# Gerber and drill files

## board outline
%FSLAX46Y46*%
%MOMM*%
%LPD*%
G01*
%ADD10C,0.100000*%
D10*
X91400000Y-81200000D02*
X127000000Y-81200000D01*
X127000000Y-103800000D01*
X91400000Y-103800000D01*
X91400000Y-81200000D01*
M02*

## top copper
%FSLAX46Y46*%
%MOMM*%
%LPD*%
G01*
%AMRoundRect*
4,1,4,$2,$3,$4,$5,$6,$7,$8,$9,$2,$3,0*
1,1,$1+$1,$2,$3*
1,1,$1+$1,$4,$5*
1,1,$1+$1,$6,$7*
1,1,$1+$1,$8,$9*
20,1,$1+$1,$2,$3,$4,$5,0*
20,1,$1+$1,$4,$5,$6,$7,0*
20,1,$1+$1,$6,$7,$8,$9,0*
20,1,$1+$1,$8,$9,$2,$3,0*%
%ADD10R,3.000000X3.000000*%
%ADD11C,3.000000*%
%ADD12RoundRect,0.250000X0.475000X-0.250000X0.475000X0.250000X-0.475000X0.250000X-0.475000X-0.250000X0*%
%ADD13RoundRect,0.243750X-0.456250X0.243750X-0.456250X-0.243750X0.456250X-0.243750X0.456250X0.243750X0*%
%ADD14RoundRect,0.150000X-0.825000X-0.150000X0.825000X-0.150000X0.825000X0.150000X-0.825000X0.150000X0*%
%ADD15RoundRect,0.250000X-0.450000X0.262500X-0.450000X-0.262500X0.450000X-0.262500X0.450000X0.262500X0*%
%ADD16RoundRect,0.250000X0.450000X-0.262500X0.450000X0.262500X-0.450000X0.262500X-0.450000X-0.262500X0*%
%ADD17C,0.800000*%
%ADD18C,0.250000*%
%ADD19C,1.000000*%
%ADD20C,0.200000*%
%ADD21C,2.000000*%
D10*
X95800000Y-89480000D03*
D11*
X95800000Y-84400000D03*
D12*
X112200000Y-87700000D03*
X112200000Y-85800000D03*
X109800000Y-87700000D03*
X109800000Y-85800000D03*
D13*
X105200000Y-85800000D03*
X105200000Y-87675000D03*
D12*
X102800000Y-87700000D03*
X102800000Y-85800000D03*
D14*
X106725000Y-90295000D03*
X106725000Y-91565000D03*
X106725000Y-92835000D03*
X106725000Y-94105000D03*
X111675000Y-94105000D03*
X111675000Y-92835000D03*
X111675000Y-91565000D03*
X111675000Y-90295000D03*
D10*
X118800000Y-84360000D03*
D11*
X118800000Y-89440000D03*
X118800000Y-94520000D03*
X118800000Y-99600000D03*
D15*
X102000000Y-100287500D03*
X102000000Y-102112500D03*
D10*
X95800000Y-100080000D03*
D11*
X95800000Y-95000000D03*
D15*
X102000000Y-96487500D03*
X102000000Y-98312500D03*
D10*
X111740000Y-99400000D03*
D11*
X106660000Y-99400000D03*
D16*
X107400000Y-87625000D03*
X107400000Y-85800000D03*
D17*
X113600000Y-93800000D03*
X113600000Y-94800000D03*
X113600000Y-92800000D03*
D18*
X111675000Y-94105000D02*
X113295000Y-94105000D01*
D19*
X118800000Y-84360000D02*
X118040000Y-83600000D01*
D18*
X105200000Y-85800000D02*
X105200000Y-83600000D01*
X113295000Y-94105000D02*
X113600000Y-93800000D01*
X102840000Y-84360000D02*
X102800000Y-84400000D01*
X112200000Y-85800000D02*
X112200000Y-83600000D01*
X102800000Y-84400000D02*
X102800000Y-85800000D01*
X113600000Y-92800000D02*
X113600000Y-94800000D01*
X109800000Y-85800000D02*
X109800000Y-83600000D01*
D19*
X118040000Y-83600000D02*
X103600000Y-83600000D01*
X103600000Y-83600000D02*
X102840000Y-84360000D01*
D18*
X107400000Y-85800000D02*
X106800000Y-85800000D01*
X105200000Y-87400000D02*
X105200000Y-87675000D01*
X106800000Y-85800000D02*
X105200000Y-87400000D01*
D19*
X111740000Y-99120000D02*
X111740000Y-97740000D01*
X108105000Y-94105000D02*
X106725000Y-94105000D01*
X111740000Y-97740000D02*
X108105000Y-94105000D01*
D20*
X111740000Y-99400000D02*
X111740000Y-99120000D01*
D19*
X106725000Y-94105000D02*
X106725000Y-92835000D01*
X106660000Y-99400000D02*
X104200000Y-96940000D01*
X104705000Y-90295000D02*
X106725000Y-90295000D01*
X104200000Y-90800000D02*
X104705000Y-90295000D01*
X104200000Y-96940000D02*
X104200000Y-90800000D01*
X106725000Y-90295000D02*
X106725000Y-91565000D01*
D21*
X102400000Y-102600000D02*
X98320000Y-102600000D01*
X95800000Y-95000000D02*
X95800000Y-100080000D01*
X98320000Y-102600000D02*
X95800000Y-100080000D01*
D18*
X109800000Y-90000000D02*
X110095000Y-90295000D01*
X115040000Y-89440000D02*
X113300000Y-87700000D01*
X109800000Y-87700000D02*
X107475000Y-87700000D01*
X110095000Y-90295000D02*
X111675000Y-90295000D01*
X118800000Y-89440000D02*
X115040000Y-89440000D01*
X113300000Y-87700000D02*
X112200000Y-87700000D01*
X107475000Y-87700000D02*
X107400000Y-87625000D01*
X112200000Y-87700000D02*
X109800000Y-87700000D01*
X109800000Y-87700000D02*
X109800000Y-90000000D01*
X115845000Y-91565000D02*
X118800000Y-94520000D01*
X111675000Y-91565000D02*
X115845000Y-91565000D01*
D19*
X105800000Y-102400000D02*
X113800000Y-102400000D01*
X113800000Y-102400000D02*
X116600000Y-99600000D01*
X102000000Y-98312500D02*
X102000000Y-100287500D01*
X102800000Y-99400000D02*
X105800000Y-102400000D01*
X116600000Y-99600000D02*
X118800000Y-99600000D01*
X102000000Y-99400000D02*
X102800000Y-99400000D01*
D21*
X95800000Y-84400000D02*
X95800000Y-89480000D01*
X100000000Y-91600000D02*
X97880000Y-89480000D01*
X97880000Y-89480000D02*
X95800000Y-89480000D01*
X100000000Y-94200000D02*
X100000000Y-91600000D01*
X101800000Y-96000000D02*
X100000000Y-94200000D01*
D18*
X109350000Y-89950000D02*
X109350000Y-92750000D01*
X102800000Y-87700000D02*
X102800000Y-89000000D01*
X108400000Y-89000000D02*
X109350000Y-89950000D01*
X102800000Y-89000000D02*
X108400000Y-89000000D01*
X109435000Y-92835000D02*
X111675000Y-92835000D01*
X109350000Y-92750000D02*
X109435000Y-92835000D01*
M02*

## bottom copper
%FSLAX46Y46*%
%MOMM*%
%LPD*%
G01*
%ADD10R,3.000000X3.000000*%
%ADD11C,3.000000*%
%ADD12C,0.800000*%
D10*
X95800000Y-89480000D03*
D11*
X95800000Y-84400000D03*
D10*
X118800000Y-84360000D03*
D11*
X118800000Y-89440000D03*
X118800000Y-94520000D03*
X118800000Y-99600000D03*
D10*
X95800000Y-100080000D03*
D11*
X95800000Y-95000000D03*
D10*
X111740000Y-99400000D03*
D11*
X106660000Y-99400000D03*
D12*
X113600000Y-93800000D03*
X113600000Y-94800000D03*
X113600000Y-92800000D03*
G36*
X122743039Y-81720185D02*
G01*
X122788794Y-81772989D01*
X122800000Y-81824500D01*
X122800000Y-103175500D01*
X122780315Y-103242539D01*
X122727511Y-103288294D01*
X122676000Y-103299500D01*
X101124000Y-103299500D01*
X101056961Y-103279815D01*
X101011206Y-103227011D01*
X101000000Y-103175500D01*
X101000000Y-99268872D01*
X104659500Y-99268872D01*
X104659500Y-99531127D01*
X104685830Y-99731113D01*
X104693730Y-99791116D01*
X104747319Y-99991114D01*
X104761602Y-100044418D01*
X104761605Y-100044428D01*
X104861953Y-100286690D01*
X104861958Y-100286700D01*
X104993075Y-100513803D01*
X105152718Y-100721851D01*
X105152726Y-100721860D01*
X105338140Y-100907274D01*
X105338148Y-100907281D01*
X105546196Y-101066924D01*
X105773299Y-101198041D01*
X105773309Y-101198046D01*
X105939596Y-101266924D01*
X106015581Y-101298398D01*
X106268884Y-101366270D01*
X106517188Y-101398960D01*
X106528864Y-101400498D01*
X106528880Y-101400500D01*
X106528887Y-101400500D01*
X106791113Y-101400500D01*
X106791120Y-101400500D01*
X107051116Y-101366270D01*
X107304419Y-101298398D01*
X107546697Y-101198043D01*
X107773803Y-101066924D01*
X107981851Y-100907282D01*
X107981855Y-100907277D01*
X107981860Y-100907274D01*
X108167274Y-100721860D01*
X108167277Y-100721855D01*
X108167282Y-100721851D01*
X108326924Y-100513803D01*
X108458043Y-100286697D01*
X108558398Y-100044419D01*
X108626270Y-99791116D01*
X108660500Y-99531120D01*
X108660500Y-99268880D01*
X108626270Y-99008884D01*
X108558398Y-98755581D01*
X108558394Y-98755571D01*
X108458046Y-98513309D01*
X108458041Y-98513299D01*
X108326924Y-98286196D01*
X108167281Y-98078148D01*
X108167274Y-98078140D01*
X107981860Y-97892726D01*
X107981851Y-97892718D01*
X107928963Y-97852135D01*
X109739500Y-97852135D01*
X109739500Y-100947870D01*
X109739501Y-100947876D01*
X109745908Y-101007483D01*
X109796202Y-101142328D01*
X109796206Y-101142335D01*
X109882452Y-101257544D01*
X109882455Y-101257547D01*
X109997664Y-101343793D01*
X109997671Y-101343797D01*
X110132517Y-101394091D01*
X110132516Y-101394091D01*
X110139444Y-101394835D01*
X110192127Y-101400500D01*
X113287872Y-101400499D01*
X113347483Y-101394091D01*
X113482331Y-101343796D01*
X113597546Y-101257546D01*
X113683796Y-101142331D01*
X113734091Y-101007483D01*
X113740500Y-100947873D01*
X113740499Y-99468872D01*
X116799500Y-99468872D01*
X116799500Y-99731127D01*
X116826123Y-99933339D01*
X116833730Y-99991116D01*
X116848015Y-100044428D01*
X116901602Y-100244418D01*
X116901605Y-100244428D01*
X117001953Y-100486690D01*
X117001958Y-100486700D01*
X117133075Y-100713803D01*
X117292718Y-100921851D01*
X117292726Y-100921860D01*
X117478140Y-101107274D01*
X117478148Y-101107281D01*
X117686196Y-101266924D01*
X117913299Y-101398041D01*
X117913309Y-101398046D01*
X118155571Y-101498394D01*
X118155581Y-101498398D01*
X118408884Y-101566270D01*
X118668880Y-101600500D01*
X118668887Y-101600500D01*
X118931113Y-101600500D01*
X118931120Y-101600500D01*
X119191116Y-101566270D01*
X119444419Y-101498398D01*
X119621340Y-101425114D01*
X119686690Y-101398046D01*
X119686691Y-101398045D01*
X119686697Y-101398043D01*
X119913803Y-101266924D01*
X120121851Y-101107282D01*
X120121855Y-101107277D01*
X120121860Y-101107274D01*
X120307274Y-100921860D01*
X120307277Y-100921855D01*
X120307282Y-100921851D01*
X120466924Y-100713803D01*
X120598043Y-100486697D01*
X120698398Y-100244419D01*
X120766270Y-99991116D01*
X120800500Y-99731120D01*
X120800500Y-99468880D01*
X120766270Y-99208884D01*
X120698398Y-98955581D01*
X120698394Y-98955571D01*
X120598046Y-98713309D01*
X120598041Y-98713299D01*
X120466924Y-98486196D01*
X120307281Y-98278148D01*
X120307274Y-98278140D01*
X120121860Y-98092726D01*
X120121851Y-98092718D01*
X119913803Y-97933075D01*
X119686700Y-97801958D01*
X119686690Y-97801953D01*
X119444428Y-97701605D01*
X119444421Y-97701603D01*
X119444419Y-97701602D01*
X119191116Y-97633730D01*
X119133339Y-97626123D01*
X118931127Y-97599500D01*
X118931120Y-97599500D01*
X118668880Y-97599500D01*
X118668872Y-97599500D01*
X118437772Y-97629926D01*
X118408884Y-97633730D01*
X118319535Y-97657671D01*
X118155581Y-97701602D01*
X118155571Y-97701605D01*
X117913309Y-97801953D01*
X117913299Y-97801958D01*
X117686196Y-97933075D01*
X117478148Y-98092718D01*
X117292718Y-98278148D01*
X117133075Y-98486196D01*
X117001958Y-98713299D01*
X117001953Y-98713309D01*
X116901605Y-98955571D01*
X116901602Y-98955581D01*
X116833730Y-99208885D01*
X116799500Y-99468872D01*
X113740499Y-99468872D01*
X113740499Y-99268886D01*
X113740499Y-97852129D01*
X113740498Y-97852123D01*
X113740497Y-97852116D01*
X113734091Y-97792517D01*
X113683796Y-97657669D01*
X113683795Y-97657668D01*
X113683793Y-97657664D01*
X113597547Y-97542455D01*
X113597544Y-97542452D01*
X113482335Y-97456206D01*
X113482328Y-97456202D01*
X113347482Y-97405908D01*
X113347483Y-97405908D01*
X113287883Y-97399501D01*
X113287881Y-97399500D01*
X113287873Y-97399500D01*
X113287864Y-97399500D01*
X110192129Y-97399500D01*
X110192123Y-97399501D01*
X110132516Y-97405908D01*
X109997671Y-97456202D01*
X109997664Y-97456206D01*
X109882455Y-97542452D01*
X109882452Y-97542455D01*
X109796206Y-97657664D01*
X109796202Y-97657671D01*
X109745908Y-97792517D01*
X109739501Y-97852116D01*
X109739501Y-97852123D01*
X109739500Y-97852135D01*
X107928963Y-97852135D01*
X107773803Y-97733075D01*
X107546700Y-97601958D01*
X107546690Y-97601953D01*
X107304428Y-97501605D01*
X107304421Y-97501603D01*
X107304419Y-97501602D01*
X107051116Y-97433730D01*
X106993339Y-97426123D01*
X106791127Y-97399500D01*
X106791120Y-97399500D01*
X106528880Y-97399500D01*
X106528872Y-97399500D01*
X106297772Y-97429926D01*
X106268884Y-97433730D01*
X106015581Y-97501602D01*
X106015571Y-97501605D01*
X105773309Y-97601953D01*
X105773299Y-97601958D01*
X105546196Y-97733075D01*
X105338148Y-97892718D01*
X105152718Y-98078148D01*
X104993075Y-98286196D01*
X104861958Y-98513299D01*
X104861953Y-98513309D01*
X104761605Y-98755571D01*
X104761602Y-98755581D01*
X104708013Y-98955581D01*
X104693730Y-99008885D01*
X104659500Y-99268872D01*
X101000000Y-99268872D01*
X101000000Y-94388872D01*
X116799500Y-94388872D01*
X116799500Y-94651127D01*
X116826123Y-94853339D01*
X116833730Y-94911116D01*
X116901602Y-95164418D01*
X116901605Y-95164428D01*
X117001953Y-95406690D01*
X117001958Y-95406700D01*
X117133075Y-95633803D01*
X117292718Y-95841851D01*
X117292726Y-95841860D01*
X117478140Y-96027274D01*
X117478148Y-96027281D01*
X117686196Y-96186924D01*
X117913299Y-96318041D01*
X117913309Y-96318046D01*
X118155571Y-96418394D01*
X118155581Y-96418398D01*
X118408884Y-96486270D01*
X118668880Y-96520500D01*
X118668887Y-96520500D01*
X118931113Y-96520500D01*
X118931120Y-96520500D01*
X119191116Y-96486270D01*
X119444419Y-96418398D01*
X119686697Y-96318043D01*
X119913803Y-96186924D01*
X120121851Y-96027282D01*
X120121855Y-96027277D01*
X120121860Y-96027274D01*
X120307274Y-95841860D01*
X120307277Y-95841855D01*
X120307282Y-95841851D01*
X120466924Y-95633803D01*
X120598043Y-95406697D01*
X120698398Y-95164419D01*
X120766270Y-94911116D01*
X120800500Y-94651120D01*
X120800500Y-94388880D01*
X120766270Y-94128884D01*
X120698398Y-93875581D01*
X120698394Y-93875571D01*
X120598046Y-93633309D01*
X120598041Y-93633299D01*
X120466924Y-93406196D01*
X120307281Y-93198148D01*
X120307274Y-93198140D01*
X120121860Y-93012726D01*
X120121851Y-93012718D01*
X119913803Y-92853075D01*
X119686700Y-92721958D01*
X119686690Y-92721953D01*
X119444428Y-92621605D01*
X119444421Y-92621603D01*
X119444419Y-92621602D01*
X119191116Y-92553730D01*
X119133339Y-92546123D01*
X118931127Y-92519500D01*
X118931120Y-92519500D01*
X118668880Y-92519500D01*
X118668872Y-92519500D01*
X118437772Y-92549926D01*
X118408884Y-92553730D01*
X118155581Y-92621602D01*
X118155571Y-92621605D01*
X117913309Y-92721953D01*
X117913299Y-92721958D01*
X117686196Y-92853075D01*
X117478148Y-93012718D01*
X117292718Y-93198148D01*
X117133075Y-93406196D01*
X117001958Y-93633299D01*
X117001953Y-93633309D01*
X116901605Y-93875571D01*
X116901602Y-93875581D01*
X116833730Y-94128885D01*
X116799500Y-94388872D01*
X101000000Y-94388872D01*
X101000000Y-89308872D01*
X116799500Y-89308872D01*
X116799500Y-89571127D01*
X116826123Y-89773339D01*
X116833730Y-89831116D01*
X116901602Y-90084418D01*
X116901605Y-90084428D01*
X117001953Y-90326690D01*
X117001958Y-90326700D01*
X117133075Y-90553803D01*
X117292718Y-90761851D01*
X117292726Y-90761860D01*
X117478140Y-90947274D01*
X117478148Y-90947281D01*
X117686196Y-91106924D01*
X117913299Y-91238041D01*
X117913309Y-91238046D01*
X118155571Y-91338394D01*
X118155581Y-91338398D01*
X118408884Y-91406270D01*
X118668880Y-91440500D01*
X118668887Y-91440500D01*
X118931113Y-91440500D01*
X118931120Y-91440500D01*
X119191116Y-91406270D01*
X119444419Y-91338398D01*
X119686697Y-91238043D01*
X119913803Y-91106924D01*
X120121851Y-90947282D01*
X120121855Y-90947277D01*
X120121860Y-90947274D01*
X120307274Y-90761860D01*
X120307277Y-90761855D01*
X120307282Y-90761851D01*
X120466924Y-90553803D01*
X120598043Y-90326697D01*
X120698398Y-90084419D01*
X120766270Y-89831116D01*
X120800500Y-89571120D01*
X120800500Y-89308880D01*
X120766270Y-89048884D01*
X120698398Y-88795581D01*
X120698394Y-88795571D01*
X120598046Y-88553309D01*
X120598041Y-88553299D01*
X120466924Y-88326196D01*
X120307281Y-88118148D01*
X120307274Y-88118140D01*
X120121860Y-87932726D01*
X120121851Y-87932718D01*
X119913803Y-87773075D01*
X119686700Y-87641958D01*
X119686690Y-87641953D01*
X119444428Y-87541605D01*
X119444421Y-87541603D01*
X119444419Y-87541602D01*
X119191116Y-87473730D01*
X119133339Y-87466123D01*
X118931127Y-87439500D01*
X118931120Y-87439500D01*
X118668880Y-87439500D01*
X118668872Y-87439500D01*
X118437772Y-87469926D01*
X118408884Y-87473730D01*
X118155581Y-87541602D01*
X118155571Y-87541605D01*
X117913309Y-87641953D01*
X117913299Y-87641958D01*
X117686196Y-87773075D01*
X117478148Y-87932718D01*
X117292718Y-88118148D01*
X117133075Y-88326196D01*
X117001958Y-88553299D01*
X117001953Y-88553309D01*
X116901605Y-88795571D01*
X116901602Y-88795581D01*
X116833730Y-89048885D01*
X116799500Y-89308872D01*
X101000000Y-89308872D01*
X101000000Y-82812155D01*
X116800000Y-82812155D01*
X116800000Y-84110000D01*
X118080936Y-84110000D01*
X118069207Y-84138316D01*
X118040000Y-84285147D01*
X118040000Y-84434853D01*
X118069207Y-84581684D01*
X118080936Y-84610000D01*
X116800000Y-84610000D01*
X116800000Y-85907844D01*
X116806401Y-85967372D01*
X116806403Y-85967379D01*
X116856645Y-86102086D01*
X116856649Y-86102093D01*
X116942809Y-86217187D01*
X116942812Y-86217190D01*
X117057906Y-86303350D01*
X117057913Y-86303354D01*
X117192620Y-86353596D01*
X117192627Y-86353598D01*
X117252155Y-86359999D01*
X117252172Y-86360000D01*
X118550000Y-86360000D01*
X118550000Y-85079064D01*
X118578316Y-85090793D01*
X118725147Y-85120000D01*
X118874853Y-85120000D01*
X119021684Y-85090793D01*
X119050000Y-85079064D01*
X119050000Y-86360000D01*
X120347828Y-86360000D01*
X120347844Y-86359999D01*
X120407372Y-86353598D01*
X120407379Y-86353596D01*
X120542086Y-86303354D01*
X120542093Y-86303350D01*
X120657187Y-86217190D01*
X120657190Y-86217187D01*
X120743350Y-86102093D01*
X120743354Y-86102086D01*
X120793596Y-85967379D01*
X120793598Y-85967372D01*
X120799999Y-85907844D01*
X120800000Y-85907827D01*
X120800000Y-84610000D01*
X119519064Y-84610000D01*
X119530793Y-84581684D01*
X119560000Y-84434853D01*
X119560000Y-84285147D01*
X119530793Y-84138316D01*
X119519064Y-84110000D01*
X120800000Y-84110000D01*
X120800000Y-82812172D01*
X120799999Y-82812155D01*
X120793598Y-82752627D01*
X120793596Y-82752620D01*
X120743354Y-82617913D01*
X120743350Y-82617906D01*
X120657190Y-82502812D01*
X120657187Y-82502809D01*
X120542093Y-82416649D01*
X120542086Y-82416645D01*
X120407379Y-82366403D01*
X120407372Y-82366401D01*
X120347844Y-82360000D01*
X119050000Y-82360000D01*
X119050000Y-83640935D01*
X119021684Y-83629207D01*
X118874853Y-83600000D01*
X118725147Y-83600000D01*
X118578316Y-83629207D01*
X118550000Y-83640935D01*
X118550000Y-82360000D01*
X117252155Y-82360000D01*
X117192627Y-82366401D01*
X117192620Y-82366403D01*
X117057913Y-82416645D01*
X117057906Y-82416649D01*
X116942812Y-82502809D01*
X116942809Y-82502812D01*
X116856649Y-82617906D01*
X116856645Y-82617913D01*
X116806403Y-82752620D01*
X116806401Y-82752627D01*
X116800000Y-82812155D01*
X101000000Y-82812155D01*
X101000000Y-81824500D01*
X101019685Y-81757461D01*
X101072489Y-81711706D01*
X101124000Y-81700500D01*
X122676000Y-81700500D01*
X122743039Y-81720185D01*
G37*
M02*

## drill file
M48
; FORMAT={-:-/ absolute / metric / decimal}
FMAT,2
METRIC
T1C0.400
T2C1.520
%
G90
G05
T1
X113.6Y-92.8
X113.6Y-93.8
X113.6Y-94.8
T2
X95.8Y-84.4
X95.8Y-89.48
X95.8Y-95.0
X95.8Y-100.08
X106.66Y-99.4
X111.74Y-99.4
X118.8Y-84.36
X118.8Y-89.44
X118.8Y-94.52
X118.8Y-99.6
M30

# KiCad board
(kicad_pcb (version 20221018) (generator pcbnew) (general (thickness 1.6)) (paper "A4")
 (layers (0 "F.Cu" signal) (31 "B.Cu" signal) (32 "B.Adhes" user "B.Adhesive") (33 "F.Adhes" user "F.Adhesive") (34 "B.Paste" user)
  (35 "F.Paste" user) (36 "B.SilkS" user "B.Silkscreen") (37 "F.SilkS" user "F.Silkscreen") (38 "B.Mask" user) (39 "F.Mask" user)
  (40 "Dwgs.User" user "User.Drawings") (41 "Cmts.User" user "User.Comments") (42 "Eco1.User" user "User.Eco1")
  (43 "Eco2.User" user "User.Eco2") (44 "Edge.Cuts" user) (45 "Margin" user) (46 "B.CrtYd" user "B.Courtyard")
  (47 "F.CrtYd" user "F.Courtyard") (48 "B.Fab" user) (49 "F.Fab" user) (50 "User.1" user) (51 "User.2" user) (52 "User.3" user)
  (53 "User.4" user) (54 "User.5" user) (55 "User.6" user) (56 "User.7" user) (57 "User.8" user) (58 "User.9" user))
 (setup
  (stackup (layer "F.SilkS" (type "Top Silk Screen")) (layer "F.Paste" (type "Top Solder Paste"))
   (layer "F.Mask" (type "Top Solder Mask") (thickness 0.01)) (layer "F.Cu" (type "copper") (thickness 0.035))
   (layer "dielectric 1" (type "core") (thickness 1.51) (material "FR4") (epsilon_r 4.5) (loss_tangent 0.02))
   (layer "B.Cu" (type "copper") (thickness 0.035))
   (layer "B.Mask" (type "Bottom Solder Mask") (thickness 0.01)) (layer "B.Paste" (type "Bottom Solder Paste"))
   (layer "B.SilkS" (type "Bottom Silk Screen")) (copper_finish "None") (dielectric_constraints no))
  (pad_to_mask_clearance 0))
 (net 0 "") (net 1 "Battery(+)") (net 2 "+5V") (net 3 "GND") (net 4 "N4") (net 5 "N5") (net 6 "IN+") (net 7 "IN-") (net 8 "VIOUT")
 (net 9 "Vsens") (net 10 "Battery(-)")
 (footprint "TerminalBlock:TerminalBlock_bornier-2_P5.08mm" (layer "F.Cu") (at 95.8 89.48 90)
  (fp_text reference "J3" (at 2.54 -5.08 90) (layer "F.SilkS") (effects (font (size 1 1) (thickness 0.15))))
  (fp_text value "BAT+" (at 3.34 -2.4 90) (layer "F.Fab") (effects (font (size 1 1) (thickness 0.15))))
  (pad "1" thru_hole rect (at 0 0 90) (size 3 3) (drill 1.52) (layers "*.Cu" "*.Mask") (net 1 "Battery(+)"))
  (pad "2" thru_hole circle (at 5.08 0 90) (size 3 3) (drill 1.52) (layers "*.Cu" "*.Mask") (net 1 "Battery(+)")))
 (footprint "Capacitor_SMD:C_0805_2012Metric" (layer "F.Cu") (at 112.2 86.75 90)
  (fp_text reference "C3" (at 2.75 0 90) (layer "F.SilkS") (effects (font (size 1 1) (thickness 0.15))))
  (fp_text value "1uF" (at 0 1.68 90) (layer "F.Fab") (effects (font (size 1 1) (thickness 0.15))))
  (pad "1" smd roundrect (at -0.95 0 90) (size 1 1.45) (layers "F.Cu" "F.Paste" "F.Mask") (roundrect_rratio 0.25) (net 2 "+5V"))
  (pad "2" smd roundrect (at 0.95 0 90) (size 1 1.45) (layers "F.Cu" "F.Paste" "F.Mask") (roundrect_rratio 0.25) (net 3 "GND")))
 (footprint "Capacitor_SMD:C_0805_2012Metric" (layer "F.Cu") (at 109.8 86.75 90)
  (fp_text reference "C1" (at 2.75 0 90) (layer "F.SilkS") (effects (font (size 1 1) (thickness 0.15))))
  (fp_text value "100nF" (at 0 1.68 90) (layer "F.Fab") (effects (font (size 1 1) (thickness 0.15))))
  (pad "1" smd roundrect (at -0.95 0 90) (size 1 1.45) (layers "F.Cu" "F.Paste" "F.Mask") (roundrect_rratio 0.25) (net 2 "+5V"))
  (pad "2" smd roundrect (at 0.95 0 90) (size 1 1.45) (layers "F.Cu" "F.Paste" "F.Mask") (roundrect_rratio 0.25) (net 3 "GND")))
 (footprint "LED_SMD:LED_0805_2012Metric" (layer "F.Cu") (at 105.2 86.7375 -90)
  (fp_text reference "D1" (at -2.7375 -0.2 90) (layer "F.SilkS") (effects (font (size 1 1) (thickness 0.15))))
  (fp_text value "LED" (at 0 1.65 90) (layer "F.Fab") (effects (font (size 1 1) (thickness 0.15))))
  (pad "1" smd roundrect (at -0.9375 0 270) (size 0.975 1.4) (layers "F.Cu" "F.Paste" "F.Mask") (roundrect_rratio 0.25) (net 3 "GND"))
  (pad "2" smd roundrect (at 0.9375 0 270) (size 0.975 1.4) (layers "F.Cu" "F.Paste" "F.Mask") (roundrect_rratio 0.25) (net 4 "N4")))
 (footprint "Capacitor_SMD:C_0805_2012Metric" (layer "F.Cu") (at 102.8 86.75 90)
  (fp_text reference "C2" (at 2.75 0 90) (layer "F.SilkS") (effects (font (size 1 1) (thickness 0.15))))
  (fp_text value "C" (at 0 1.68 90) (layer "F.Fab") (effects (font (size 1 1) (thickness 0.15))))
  (pad "1" smd roundrect (at -0.95 0 90) (size 1 1.45) (layers "F.Cu" "F.Paste" "F.Mask") (roundrect_rratio 0.25) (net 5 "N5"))
  (pad "2" smd roundrect (at 0.95 0 90) (size 1 1.45) (layers "F.Cu" "F.Paste" "F.Mask") (roundrect_rratio 0.25) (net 3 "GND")))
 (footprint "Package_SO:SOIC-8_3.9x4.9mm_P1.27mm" (layer "F.Cu") (at 109.2 92.2)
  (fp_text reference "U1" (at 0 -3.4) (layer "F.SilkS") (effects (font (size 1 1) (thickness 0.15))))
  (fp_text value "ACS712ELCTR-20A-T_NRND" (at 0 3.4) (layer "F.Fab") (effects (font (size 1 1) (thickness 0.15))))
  (pad "1" smd roundrect (at -2.475 -1.905) (size 1.95 0.6) (layers "F.Cu" "F.Paste" "F.Mask") (roundrect_rratio 0.25) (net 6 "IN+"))
  (pad "2" smd roundrect (at -2.475 -0.635) (size 1.95 0.6) (layers "F.Cu" "F.Paste" "F.Mask") (roundrect_rratio 0.25) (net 6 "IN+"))
  (pad "3" smd roundrect (at -2.475 0.635) (size 1.95 0.6) (layers "F.Cu" "F.Paste" "F.Mask") (roundrect_rratio 0.25) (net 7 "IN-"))
  (pad "4" smd roundrect (at -2.475 1.905) (size 1.95 0.6) (layers "F.Cu" "F.Paste" "F.Mask") (roundrect_rratio 0.25) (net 7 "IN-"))
  (pad "5" smd roundrect (at 2.475 1.905) (size 1.95 0.6) (layers "F.Cu" "F.Paste" "F.Mask") (roundrect_rratio 0.25) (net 3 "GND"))
  (pad "6" smd roundrect (at 2.475 0.635) (size 1.95 0.6) (layers "F.Cu" "F.Paste" "F.Mask") (roundrect_rratio 0.25) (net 5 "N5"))
  (pad "7" smd roundrect (at 2.475 -0.635) (size 1.95 0.6) (layers "F.Cu" "F.Paste" "F.Mask") (roundrect_rratio 0.25) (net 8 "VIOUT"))
  (pad "8" smd roundrect (at 2.475 -1.905) (size 1.95 0.6) (layers "F.Cu" "F.Paste" "F.Mask") (roundrect_rratio 0.25) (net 2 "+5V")))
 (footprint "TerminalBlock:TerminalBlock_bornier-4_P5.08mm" (layer "F.Cu") (at 118.8 84.36 -90)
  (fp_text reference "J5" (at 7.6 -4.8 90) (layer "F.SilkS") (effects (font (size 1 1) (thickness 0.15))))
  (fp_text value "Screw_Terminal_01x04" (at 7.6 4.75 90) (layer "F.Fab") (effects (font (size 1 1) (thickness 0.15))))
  (pad "1" thru_hole rect (at 0 0 270) (size 3 3) (drill 1.52) (layers "*.Cu" "*.Mask") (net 3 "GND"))
  (pad "2" thru_hole circle (at 5.08 0 270) (size 3 3) (drill 1.52) (layers "*.Cu" "*.Mask") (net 2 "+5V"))
  (pad "3" thru_hole circle (at 10.16 0 270) (size 3 3) (drill 1.52) (layers "*.Cu" "*.Mask") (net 8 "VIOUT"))
  (pad "4" thru_hole circle (at 15.24 0 270) (size 3 3) (drill 1.52) (layers "*.Cu" "*.Mask") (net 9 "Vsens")))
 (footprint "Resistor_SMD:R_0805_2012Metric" (layer "F.Cu") (at 102 101.2 -90)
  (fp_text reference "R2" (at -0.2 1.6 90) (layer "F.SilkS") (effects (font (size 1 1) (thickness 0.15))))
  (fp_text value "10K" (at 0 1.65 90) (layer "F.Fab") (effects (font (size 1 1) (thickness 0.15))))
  (pad "1" smd roundrect (at -0.9125 0 270) (size 1.025 1.4) (layers "F.Cu" "F.Paste" "F.Mask") (roundrect_rratio 0.243902) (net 9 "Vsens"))
  (pad "2" smd roundrect (at 0.9125 0 270) (size 1.025 1.4) (layers "F.Cu" "F.Paste" "F.Mask") (roundrect_rratio 0.243902)
   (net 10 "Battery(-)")))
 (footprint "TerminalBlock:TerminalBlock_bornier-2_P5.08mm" (layer "F.Cu") (at 95.8 100.08 90)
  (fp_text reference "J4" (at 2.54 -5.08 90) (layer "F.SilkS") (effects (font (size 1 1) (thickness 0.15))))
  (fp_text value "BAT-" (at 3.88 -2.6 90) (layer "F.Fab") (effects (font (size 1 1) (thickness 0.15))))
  (pad "1" thru_hole rect (at 0 0 90) (size 3 3) (drill 1.52) (layers "*.Cu" "*.Mask") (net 10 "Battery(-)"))
  (pad "2" thru_hole circle (at 5.08 0 90) (size 3 3) (drill 1.52) (layers "*.Cu" "*.Mask") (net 10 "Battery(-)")))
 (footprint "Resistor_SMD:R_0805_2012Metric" (layer "F.Cu") (at 102 97.4 -90)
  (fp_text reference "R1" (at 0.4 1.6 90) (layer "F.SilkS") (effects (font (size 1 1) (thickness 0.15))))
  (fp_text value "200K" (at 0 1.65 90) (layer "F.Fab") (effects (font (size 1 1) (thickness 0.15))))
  (pad "1" smd roundrect (at -0.9125 0 270) (size 1.025 1.4) (layers "F.Cu" "F.Paste" "F.Mask") (roundrect_rratio 0.243902)
   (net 1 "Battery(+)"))
  (pad "2" smd roundrect (at 0.9125 0 270) (size 1.025 1.4) (layers "F.Cu" "F.Paste" "F.Mask") (roundrect_rratio 0.243902) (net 9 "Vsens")))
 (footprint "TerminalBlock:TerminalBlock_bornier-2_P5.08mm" (layer "F.Cu") (at 111.74 99.4 180)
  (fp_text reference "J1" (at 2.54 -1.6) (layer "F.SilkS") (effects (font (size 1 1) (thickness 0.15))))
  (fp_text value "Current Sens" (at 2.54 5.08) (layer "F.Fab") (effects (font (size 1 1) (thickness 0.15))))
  (pad "1" thru_hole rect (at 0 0 180) (size 3 3) (drill 1.52) (layers "*.Cu" "*.Mask") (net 7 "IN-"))
  (pad "2" thru_hole circle (at 5.08 0 180) (size 3 3) (drill 1.52) (layers "*.Cu" "*.Mask") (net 6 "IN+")))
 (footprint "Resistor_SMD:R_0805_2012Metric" (layer "F.Cu") (at 107.4 86.7125 90)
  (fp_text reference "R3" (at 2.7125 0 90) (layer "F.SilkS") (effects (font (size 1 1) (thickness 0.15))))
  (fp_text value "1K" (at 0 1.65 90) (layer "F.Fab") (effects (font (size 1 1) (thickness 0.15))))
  (pad "1" smd roundrect (at -0.9125 0 90) (size 1.025 1.4) (layers "F.Cu" "F.Paste" "F.Mask") (roundrect_rratio 0.243902) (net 2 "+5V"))
  (pad "2" smd roundrect (at 0.9125 0 90) (size 1.025 1.4) (layers "F.Cu" "F.Paste" "F.Mask") (roundrect_rratio 0.243902) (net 4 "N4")))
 (gr_rect (start 91.4 81.2) (end 127 103.8) (stroke (width 0.1) (type default)) (fill none) (layer "Edge.Cuts"))
 (segment (start 111.675 94.105) (end 113.295 94.105) (width 0.25) (layer "F.Cu") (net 3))
 (segment (start 118.8 84.36) (end 118.04 83.6) (width 1) (layer "F.Cu") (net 3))
 (segment (start 105.2 85.8) (end 105.2 83.6) (width 0.25) (layer "F.Cu") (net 3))
 (segment (start 113.295 94.105) (end 113.6 93.8) (width 0.25) (layer "F.Cu") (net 3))
 (segment (start 102.84 84.36) (end 102.8 84.4) (width 0.25) (layer "F.Cu") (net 3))
 (segment (start 112.2 85.8) (end 112.2 83.6) (width 0.25) (layer "F.Cu") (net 3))
 (segment (start 102.8 84.4) (end 102.8 85.8) (width 0.25) (layer "F.Cu") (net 3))
 (segment (start 113.6 92.8) (end 113.6 94.8) (width 0.25) (layer "F.Cu") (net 3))
 (segment (start 109.8 85.8) (end 109.8 83.6) (width 0.25) (layer "F.Cu") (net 3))
 (segment (start 118.04 83.6) (end 103.6 83.6) (width 1) (layer "F.Cu") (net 3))
 (segment (start 103.6 83.6) (end 102.84 84.36) (width 1) (layer "F.Cu") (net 3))
 (via (at 113.6 93.8) (size 0.8) (drill 0.4) (layers "F.Cu" "B.Cu") (free) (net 3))
 (via (at 113.6 94.8) (size 0.8) (drill 0.4) (layers "F.Cu" "B.Cu") (free) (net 3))
 (via (at 113.6 92.8) (size 0.8) (drill 0.4) (layers "F.Cu" "B.Cu") (free) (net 3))
 (segment (start 107.4 85.8) (end 106.8 85.8) (width 0.25) (layer "F.Cu") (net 4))
 (segment (start 105.2 87.4) (end 105.2 87.675) (width 0.25) (layer "F.Cu") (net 4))
 (segment (start 106.8 85.8) (end 105.2 87.4) (width 0.25) (layer "F.Cu") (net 4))
 (segment (start 111.74 99.12) (end 111.74 97.74) (width 1) (layer "F.Cu") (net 7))
 (segment (start 108.105 94.105) (end 106.725 94.105) (width 1) (layer "F.Cu") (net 7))
 (segment (start 111.74 97.74) (end 108.105 94.105) (width 1) (layer "F.Cu") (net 7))
 (segment (start 111.74 99.4) (end 111.74 99.12) (width 0.2) (layer "F.Cu") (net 7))
 (segment (start 106.725 94.105) (end 106.725 92.835) (width 1) (layer "F.Cu") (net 7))
 (segment (start 106.66 99.4) (end 104.2 96.94) (width 1) (layer "F.Cu") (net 6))
 (segment (start 104.705 90.295) (end 106.725 90.295) (width 1) (layer "F.Cu") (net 6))
 (segment (start 104.2 90.8) (end 104.705 90.295) (width 1) (layer "F.Cu") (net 6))
 (segment (start 104.2 96.94) (end 104.2 90.8) (width 1) (layer "F.Cu") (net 6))
 (segment (start 106.725 90.295) (end 106.725 91.565) (width 1) (layer "F.Cu") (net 6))
 (segment (start 102.4 102.6) (end 98.32 102.6) (width 2) (layer "F.Cu") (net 10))
 (segment (start 95.8 95) (end 95.8 100.08) (width 2) (layer "F.Cu") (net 10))
 (segment (start 98.32 102.6) (end 95.8 100.08) (width 2) (layer "F.Cu") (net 10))
 (segment (start 109.8 90) (end 110.095 90.295) (width 0.25) (layer "F.Cu") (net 2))
 (segment (start 115.04 89.44) (end 113.3 87.7) (width 0.25) (layer "F.Cu") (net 2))
 (segment (start 109.8 87.7) (end 107.475 87.7) (width 0.25) (layer "F.Cu") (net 2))
 (segment (start 110.095 90.295) (end 111.675 90.295) (width 0.25) (layer "F.Cu") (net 2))
 (segment (start 118.8 89.44) (end 115.04 89.44) (width 0.25) (layer "F.Cu") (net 2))
 (segment (start 113.3 87.7) (end 112.2 87.7) (width 0.25) (layer "F.Cu") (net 2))
 (segment (start 107.475 87.7) (end 107.4 87.625) (width 0.25) (layer "F.Cu") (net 2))
 (segment (start 112.2 87.7) (end 109.8 87.7) (width 0.25) (layer "F.Cu") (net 2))
 (segment (start 109.8 87.7) (end 109.8 90) (width 0.25) (layer "F.Cu") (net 2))
 (segment (start 115.845 91.565) (end 118.8 94.52) (width 0.25) (layer "F.Cu") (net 8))
 (segment (start 111.675 91.565) (end 115.845 91.565) (width 0.25) (layer "F.Cu") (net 8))
 (segment (start 105.8 102.4) (end 113.8 102.4) (width 1) (layer "F.Cu") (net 9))
 (segment (start 113.8 102.4) (end 116.6 99.6) (width 1) (layer "F.Cu") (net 9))
 (segment (start 102 98.3125) (end 102 100.2875) (width 1) (layer "F.Cu") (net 9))
 (segment (start 102.8 99.4) (end 105.8 102.4) (width 1) (layer "F.Cu") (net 9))
 (segment (start 116.6 99.6) (end 118.8 99.6) (width 1) (layer "F.Cu") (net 9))
 (segment (start 102 99.4) (end 102.8 99.4) (width 1) (layer "F.Cu") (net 9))
 (segment (start 95.8 84.4) (end 95.8 89.48) (width 2) (layer "F.Cu") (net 1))
 (segment (start 100 91.6) (end 97.88 89.48) (width 2) (layer "F.Cu") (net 1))
 (segment (start 97.88 89.48) (end 95.8 89.48) (width 2) (layer "F.Cu") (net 1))
 (segment (start 100 94.2) (end 100 91.6) (width 2) (layer "F.Cu") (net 1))
 (segment (start 101.8 96) (end 100 94.2) (width 2) (layer "F.Cu") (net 1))
 (segment (start 109.35 89.95) (end 109.35 92.75) (width 0.25) (layer "F.Cu") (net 5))
 (segment (start 102.8 87.7) (end 102.8 89) (width 0.25) (layer "F.Cu") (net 5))
 (segment (start 108.4 89) (end 109.35 89.95) (width 0.25) (layer "F.Cu") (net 5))
 (segment (start 102.8 89) (end 108.4 89) (width 0.25) (layer "F.Cu") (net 5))
 (segment (start 109.435 92.835) (end 111.675 92.835) (width 0.25) (layer "F.Cu") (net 5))
 (segment (start 109.35 92.75) (end 109.435 92.835) (width 0.25) (layer "F.Cu") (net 5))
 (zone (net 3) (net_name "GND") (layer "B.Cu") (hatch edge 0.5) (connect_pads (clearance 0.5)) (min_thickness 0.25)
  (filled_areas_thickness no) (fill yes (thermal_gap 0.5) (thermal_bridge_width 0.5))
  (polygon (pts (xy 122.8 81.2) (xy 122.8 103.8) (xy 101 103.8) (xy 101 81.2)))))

